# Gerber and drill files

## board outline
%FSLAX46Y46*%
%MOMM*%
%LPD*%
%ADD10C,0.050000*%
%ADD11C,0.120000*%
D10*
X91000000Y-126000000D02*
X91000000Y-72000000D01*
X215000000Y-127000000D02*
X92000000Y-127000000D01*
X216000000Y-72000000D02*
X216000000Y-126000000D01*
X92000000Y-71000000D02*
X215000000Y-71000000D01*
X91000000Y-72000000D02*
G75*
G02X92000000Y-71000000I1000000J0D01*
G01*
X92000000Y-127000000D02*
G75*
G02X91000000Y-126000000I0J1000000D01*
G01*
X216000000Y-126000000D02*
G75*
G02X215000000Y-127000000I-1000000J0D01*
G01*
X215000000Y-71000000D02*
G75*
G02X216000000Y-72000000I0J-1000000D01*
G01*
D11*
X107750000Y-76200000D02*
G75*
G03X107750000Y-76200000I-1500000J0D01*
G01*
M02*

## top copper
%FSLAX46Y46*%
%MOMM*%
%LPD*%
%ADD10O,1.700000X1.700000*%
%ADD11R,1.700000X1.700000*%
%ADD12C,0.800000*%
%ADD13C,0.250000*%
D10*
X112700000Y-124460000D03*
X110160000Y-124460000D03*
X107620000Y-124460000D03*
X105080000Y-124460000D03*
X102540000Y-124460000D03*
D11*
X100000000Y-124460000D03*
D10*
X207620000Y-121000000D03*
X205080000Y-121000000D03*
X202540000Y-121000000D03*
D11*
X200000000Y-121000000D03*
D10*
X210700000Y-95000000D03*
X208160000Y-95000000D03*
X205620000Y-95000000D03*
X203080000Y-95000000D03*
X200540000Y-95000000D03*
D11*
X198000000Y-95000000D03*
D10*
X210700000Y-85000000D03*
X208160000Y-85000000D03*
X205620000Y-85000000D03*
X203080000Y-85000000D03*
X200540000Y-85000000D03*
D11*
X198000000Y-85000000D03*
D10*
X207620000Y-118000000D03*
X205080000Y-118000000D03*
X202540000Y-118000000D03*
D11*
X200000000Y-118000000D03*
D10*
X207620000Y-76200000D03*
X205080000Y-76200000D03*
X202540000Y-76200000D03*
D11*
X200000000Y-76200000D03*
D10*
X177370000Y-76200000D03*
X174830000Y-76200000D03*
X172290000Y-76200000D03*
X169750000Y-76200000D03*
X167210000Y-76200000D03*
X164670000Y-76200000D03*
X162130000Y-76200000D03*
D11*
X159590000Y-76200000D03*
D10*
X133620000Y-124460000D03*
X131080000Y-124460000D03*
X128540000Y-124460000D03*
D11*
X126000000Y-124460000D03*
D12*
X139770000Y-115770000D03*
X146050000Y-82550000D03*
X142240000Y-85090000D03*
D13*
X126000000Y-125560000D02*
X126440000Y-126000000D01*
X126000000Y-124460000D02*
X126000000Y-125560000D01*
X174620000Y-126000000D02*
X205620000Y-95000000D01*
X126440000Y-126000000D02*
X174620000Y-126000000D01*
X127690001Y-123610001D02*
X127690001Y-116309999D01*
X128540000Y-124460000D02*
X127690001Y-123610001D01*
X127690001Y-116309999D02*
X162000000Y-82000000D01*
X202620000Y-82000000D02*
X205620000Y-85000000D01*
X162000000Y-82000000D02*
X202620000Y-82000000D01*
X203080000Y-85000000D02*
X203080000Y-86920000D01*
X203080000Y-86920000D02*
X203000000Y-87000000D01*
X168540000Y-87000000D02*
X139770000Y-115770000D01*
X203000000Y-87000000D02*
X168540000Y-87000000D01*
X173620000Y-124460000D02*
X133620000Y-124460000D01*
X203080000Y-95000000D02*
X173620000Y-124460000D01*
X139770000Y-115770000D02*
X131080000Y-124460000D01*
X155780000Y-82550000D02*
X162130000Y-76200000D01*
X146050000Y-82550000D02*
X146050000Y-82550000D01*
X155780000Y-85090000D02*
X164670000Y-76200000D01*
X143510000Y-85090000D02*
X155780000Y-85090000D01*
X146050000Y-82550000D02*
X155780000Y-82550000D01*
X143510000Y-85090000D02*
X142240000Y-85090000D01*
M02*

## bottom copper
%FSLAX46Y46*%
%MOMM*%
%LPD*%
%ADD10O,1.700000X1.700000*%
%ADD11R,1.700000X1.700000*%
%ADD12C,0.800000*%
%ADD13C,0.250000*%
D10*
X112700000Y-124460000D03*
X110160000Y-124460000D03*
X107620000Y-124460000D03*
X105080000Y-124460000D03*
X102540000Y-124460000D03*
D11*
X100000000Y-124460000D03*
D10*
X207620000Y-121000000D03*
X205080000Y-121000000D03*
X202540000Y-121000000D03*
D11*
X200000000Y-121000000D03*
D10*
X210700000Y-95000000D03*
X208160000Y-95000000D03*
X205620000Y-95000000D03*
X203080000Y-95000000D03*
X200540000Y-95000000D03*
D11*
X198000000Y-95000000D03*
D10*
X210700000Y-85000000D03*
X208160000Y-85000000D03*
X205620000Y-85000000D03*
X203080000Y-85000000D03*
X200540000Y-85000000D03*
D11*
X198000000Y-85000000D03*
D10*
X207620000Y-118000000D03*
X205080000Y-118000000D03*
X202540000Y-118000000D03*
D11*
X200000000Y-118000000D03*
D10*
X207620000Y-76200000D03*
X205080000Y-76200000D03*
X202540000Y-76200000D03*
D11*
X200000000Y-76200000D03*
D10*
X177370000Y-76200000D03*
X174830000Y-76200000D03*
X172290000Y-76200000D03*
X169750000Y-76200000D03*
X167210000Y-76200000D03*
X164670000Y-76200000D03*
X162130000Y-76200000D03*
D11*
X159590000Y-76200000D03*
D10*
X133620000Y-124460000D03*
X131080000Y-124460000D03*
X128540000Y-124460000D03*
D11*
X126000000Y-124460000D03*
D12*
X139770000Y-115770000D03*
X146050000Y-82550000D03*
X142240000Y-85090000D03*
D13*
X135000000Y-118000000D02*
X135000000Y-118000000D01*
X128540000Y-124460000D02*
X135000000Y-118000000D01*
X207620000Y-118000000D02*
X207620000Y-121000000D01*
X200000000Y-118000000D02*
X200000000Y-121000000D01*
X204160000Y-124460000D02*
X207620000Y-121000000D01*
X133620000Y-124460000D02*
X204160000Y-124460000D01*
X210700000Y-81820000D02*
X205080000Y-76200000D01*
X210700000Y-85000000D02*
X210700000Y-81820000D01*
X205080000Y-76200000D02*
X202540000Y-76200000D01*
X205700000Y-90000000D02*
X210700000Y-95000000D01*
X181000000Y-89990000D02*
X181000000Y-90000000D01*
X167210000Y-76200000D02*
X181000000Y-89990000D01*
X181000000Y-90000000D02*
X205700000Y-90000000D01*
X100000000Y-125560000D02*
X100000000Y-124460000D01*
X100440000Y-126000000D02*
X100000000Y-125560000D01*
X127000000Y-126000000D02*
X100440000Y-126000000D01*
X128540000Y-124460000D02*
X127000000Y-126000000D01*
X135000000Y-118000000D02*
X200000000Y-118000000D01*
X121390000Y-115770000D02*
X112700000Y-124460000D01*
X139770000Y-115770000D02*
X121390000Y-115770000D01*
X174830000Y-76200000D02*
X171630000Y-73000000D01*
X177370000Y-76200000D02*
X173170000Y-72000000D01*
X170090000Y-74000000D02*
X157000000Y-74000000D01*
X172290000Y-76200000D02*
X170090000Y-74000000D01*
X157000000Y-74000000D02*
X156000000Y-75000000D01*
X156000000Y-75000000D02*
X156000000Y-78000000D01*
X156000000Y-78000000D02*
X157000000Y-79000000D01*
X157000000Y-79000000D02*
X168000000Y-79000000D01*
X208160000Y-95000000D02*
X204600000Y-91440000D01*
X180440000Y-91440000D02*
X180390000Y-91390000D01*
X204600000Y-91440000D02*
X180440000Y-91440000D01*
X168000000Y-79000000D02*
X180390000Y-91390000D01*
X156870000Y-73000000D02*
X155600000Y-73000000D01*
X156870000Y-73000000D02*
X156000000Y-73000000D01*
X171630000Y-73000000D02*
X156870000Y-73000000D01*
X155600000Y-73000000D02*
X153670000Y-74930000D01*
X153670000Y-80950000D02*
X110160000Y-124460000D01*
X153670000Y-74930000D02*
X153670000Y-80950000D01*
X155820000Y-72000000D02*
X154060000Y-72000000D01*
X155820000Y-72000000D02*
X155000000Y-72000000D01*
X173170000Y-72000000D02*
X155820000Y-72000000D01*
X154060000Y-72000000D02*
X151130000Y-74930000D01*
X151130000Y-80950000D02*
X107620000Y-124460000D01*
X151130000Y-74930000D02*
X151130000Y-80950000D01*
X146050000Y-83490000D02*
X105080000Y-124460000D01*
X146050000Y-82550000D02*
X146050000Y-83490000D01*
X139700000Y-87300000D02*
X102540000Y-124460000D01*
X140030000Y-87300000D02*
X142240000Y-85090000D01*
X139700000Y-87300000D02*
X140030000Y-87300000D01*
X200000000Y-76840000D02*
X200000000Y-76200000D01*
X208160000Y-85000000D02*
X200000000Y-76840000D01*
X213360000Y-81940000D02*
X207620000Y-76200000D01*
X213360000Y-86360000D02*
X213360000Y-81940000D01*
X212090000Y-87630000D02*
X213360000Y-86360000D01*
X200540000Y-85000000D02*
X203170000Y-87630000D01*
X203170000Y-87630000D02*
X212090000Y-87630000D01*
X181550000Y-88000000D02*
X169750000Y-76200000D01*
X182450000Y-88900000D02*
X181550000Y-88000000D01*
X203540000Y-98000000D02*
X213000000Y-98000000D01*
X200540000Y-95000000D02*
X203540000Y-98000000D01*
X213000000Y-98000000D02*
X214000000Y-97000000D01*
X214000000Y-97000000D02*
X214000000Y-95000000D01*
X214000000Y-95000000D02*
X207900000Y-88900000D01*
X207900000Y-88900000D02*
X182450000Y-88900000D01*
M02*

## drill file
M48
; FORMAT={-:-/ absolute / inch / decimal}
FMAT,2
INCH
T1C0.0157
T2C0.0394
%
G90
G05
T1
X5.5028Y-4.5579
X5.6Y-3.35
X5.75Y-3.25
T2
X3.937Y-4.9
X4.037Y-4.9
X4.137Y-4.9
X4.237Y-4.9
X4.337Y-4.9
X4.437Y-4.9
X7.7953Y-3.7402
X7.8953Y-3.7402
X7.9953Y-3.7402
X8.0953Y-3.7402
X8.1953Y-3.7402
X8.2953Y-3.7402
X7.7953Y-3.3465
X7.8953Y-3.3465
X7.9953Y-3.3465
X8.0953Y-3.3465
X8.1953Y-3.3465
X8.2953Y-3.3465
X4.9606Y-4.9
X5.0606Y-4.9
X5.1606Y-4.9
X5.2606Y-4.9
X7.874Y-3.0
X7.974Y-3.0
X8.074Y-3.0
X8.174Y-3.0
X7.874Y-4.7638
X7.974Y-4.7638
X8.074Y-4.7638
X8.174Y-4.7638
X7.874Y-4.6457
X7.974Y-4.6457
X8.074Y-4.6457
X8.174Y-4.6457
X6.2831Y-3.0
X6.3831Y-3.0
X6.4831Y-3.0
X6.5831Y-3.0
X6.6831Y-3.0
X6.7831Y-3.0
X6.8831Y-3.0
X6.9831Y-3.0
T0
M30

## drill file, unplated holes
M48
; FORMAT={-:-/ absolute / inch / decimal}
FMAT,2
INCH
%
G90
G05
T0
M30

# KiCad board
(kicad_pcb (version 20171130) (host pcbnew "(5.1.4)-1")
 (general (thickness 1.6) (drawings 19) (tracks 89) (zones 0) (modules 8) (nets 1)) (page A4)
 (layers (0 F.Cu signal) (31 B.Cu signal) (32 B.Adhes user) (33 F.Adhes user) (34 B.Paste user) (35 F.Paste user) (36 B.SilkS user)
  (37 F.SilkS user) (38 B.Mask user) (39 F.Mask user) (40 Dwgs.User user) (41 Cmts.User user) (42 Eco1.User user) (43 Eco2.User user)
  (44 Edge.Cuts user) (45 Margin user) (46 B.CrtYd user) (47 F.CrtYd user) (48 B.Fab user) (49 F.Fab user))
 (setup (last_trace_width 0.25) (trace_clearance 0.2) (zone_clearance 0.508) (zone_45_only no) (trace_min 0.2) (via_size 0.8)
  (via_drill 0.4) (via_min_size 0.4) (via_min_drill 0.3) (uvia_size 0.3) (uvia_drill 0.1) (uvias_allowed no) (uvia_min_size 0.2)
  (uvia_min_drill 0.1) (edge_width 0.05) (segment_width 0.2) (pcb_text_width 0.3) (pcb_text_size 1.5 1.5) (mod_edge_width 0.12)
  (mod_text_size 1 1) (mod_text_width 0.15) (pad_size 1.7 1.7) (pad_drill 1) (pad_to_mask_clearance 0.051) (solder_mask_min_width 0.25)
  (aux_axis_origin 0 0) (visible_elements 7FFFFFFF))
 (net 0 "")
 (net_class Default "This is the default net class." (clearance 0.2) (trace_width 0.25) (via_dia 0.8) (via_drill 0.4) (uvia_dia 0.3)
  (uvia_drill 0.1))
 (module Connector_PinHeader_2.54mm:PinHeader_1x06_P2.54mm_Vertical (layer B.Cu) (at 100 124.46 270)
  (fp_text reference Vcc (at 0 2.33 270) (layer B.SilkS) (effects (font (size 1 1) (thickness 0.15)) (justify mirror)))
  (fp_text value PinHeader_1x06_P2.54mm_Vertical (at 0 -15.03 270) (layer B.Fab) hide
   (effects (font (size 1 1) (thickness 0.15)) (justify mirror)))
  (pad 6 thru_hole oval (at 0 -12.7 270) (size 1.7 1.7) (drill 1) (layers *.Cu *.Mask))
  (pad 5 thru_hole oval (at 0 -10.16 270) (size 1.7 1.7) (drill 1) (layers *.Cu *.Mask))
  (pad 4 thru_hole oval (at 0 -7.62 270) (size 1.7 1.7) (drill 1) (layers *.Cu *.Mask))
  (pad 3 thru_hole oval (at 0 -5.08 270) (size 1.7 1.7) (drill 1) (layers *.Cu *.Mask))
  (pad 2 thru_hole oval (at 0 -2.54 270) (size 1.7 1.7) (drill 1) (layers *.Cu *.Mask))
  (pad 1 thru_hole rect (at 0 0 270) (size 1.7 1.7) (drill 1) (layers *.Cu *.Mask)))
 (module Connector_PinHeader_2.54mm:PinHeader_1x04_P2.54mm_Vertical (layer F.Cu) (at 200 121 90)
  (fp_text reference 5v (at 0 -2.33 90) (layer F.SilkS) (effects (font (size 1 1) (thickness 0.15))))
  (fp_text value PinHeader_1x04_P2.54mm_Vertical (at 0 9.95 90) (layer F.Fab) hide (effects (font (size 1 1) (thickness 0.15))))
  (pad 4 thru_hole oval (at 0 7.62 90) (size 1.7 1.7) (drill 1) (layers *.Cu *.Mask))
  (pad 3 thru_hole oval (at 0 5.08 90) (size 1.7 1.7) (drill 1) (layers *.Cu *.Mask))
  (pad 2 thru_hole oval (at 0 2.54 90) (size 1.7 1.7) (drill 1) (layers *.Cu *.Mask))
  (pad 1 thru_hole rect (at 0 0 90) (size 1.7 1.7) (drill 1) (layers *.Cu *.Mask)))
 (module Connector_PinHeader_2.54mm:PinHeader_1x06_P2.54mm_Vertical (layer B.Cu) (at 198 95 270)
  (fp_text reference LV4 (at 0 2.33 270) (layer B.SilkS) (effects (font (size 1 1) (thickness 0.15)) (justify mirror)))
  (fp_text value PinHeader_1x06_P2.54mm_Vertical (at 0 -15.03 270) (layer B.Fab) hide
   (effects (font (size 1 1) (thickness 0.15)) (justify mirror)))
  (pad 6 thru_hole oval (at 0 -12.7 270) (size 1.7 1.7) (drill 1) (layers *.Cu *.Mask))
  (pad 5 thru_hole oval (at 0 -10.16 270) (size 1.7 1.7) (drill 1) (layers *.Cu *.Mask))
  (pad 4 thru_hole oval (at 0 -7.62 270) (size 1.7 1.7) (drill 1) (layers *.Cu *.Mask))
  (pad 3 thru_hole oval (at 0 -5.08 270) (size 1.7 1.7) (drill 1) (layers *.Cu *.Mask))
  (pad 2 thru_hole oval (at 0 -2.54 270) (size 1.7 1.7) (drill 1) (layers *.Cu *.Mask))
  (pad 1 thru_hole rect (at 0 0 270) (size 1.7 1.7) (drill 1) (layers *.Cu *.Mask)))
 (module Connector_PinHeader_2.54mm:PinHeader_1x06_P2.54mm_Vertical (layer B.Cu) (at 198 85 270)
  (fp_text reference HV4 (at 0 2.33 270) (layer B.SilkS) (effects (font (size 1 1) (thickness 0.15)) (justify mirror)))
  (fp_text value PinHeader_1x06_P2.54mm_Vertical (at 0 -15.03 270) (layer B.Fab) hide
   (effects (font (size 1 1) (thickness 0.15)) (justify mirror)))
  (pad 6 thru_hole oval (at 0 -12.7 270) (size 1.7 1.7) (drill 1) (layers *.Cu *.Mask))
  (pad 5 thru_hole oval (at 0 -10.16 270) (size 1.7 1.7) (drill 1) (layers *.Cu *.Mask))
  (pad 4 thru_hole oval (at 0 -7.62 270) (size 1.7 1.7) (drill 1) (layers *.Cu *.Mask))
  (pad 3 thru_hole oval (at 0 -5.08 270) (size 1.7 1.7) (drill 1) (layers *.Cu *.Mask))
  (pad 2 thru_hole oval (at 0 -2.54 270) (size 1.7 1.7) (drill 1) (layers *.Cu *.Mask))
  (pad 1 thru_hole rect (at 0 0 270) (size 1.7 1.7) (drill 1) (layers *.Cu *.Mask)))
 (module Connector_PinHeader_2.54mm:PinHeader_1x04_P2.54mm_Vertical (layer F.Cu) (at 200 118 90)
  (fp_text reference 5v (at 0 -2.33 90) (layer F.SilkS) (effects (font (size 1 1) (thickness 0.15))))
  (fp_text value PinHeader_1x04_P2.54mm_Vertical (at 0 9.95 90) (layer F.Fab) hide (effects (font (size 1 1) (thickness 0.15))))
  (pad 4 thru_hole oval (at 0 7.62 90) (size 1.7 1.7) (drill 1) (layers *.Cu *.Mask))
  (pad 3 thru_hole oval (at 0 5.08 90) (size 1.7 1.7) (drill 1) (layers *.Cu *.Mask))
  (pad 2 thru_hole oval (at 0 2.54 90) (size 1.7 1.7) (drill 1) (layers *.Cu *.Mask))
  (pad 1 thru_hole rect (at 0 0 90) (size 1.7 1.7) (drill 1) (layers *.Cu *.Mask)))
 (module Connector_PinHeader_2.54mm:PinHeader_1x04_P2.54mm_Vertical (layer F.Cu) (at 200 76.2 90)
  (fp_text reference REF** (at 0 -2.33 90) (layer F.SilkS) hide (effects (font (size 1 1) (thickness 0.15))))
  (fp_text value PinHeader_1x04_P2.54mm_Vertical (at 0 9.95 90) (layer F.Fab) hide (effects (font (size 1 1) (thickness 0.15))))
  (pad 4 thru_hole oval (at 0 7.62 90) (size 1.7 1.7) (drill 1) (layers *.Cu *.Mask))
  (pad 3 thru_hole oval (at 0 5.08 90) (size 1.7 1.7) (drill 1) (layers *.Cu *.Mask))
  (pad 2 thru_hole oval (at 0 2.54 90) (size 1.7 1.7) (drill 1) (layers *.Cu *.Mask))
  (pad 1 thru_hole rect (at 0 0 90) (size 1.7 1.7) (drill 1) (layers *.Cu *.Mask)))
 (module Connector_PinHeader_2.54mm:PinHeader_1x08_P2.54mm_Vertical (layer F.Cu) (at 159.59 76.2 90)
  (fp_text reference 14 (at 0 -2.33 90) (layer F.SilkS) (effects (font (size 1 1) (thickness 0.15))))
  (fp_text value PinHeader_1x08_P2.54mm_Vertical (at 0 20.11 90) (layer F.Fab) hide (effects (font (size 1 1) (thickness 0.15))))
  (pad 8 thru_hole oval (at 0 17.78 90) (size 1.7 1.7) (drill 1) (layers *.Cu *.Mask))
  (pad 7 thru_hole oval (at 0 15.24 90) (size 1.7 1.7) (drill 1) (layers *.Cu *.Mask))
  (pad 6 thru_hole oval (at 0 12.7 90) (size 1.7 1.7) (drill 1) (layers *.Cu *.Mask))
  (pad 5 thru_hole oval (at 0 10.16 90) (size 1.7 1.7) (drill 1) (layers *.Cu *.Mask))
  (pad 4 thru_hole oval (at 0 7.62 90) (size 1.7 1.7) (drill 1) (layers *.Cu *.Mask))
  (pad 3 thru_hole oval (at 0 5.08 90) (size 1.7 1.7) (drill 1) (layers *.Cu *.Mask))
  (pad 2 thru_hole oval (at 0 2.54 90) (size 1.7 1.7) (drill 1) (layers *.Cu *.Mask))
  (pad 1 thru_hole rect (at 0 0 90) (size 1.7 1.7) (drill 1) (layers *.Cu *.Mask)))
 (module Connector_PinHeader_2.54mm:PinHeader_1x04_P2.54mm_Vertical (layer F.Cu) (at 126 124.46 90)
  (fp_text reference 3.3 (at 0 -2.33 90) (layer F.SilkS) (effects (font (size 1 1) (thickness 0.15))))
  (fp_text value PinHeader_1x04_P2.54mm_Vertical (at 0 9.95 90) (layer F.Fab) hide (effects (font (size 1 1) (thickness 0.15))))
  (pad 4 thru_hole oval (at 0 7.62 90) (size 1.7 1.7) (drill 1) (layers *.Cu *.Mask))
  (pad 3 thru_hole oval (at 0 5.08 90) (size 1.7 1.7) (drill 1) (layers *.Cu *.Mask))
  (pad 2 thru_hole oval (at 0 2.54 90) (size 1.7 1.7) (drill 1) (layers *.Cu *.Mask))
  (pad 1 thru_hole rect (at 0 0 90) (size 1.7 1.7) (drill 1) (layers *.Cu *.Mask)))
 (gr_line (start 91 126) (end 91 72) (layer Edge.Cuts) (width 0.05))
 (gr_line (start 215 127) (end 92 127) (layer Edge.Cuts) (width 0.05))
 (gr_line (start 216 72) (end 216 126) (layer Edge.Cuts) (width 0.05))
 (gr_line (start 92 71) (end 215 71) (layer Edge.Cuts) (width 0.05))
 (gr_arc (start 92 72) (end 92 71) (angle -90) (layer Edge.Cuts) (width 0.05))
 (gr_arc (start 92 126) (end 91 126) (angle -90) (layer Edge.Cuts) (width 0.05))
 (gr_arc (start 215 126) (end 215 127) (angle -90) (layer Edge.Cuts) (width 0.05))
 (gr_arc (start 215 72) (end 216 72) (angle -90) (layer Edge.Cuts) (width 0.05))
 (gr_circle (center 106.25 76.2) (end 107.75 76.2) (layer Edge.Cuts) (width 0.12))
 (segment (start 126 125.56) (end 126.44 126) (width 0.25) (layer F.Cu) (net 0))
 (segment (start 126 124.46) (end 126 125.56) (width 0.25) (layer F.Cu) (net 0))
 (segment (start 174.62 126) (end 205.62 95) (width 0.25) (layer F.Cu) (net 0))
 (segment (start 126.44 126) (end 174.62 126) (width 0.25) (layer F.Cu) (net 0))
 (segment (start 127.690001 123.610001) (end 127.690001 116.309999) (width 0.25) (layer F.Cu) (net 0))
 (segment (start 128.54 124.46) (end 127.690001 123.610001) (width 0.25) (layer F.Cu) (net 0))
 (segment (start 127.690001 116.309999) (end 162 82) (width 0.25) (layer F.Cu) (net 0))
 (segment (start 202.62 82) (end 205.62 85) (width 0.25) (layer F.Cu) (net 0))
 (segment (start 162 82) (end 202.62 82) (width 0.25) (layer F.Cu) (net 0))
 (segment (start 203.08 85) (end 203.08 86.92) (width 0.25) (layer F.Cu) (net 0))
 (segment (start 203.08 86.92) (end 203 87) (width 0.25) (layer F.Cu) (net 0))
 (segment (start 168.54 87) (end 139.77 115.77) (width 0.25) (layer F.Cu) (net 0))
 (segment (start 203 87) (end 168.54 87) (width 0.25) (layer F.Cu) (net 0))
 (segment (start 173.62 124.46) (end 133.62 124.46) (width 0.25) (layer F.Cu) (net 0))
 (segment (start 203.08 95) (end 173.62 124.46) (width 0.25) (layer F.Cu) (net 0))
 (segment (start 135 118) (end 135 118) (width 0.25) (layer B.Cu) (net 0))
 (segment (start 128.54 124.46) (end 135 118) (width 0.25) (layer B.Cu) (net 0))
 (segment (start 207.62 118) (end 207.62 121) (width 0.25) (layer B.Cu) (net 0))
 (segment (start 200 118) (end 200 121) (width 0.25) (layer B.Cu) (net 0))
 (segment (start 204.16 124.46) (end 207.62 121) (width 0.25) (layer B.Cu) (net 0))
 (segment (start 133.62 124.46) (end 204.16 124.46) (width 0.25) (layer B.Cu) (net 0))
 (segment (start 210.7 81.82) (end 205.08 76.2) (width 0.25) (layer B.Cu) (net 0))
 (segment (start 210.7 85) (end 210.7 81.82) (width 0.25) (layer B.Cu) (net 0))
 (segment (start 205.08 76.2) (end 202.54 76.2) (width 0.25) (layer B.Cu) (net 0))
 (segment (start 205.7 90) (end 210.7 95) (width 0.25) (layer B.Cu) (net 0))
 (segment (start 181 89.99) (end 181 90) (width 0.25) (layer B.Cu) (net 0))
 (segment (start 167.21 76.2) (end 181 89.99) (width 0.25) (layer B.Cu) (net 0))
 (segment (start 181 90) (end 205.7 90) (width 0.25) (layer B.Cu) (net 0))
 (segment (start 100 125.56) (end 100 124.46) (width 0.25) (layer B.Cu) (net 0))
 (segment (start 100.44 126) (end 100 125.56) (width 0.25) (layer B.Cu) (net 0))
 (segment (start 127 126) (end 100.44 126) (width 0.25) (layer B.Cu) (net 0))
 (segment (start 128.54 124.46) (end 127 126) (width 0.25) (layer B.Cu) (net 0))
 (segment (start 135 118) (end 200 118) (width 0.25) (layer B.Cu) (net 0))
 (segment (start 139.77 115.77) (end 131.08 124.46) (width 0.25) (layer F.Cu) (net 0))
 (via (at 139.77 115.77) (size 0.8) (drill 0.4) (layers F.Cu B.Cu) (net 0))
 (segment (start 121.39 115.77) (end 112.7 124.46) (width 0.25) (layer B.Cu) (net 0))
 (segment (start 139.77 115.77) (end 121.39 115.77) (width 0.25) (layer B.Cu) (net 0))
 (segment (start 174.83 76.2) (end 171.63 73) (width 0.25) (layer B.Cu) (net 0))
 (segment (start 177.37 76.2) (end 173.17 72) (width 0.25) (layer B.Cu) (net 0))
 (segment (start 170.09 74) (end 157 74) (width 0.25) (layer B.Cu) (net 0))
 (segment (start 172.29 76.2) (end 170.09 74) (width 0.25) (layer B.Cu) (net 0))
 (segment (start 157 74) (end 156 75) (width 0.25) (layer B.Cu) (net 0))
 (segment (start 156 75) (end 156 78) (width 0.25) (layer B.Cu) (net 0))
 (segment (start 156 78) (end 157 79) (width 0.25) (layer B.Cu) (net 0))
 (segment (start 157 79) (end 168 79) (width 0.25) (layer B.Cu) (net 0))
 (segment (start 208.16 95) (end 204.6 91.44) (width 0.25) (layer B.Cu) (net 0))
 (segment (start 180.44 91.44) (end 180.39 91.39) (width 0.25) (layer B.Cu) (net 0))
 (segment (start 204.6 91.44) (end 180.44 91.44) (width 0.25) (layer B.Cu) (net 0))
 (segment (start 168 79) (end 180.39 91.39) (width 0.25) (layer B.Cu) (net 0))
 (segment (start 156.87 73) (end 155.6 73) (width 0.25) (layer B.Cu) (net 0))
 (segment (start 156.87 73) (end 156 73) (width 0.25) (layer B.Cu) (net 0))
 (segment (start 171.63 73) (end 156.87 73) (width 0.25) (layer B.Cu) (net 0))
 (segment (start 155.6 73) (end 153.67 74.93) (width 0.25) (layer B.Cu) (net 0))
 (segment (start 153.67 80.95) (end 110.16 124.46) (width 0.25) (layer B.Cu) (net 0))
 (segment (start 153.67 74.93) (end 153.67 80.95) (width 0.25) (layer B.Cu) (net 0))
 (segment (start 155.82 72) (end 154.06 72) (width 0.25) (layer B.Cu) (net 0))
 (segment (start 155.82 72) (end 155 72) (width 0.25) (layer B.Cu) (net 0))
 (segment (start 173.17 72) (end 155.82 72) (width 0.25) (layer B.Cu) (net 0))
 (segment (start 154.06 72) (end 151.13 74.93) (width 0.25) (layer B.Cu) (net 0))
 (segment (start 151.13 80.95) (end 107.62 124.46) (width 0.25) (layer B.Cu) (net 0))
 (segment (start 151.13 74.93) (end 151.13 80.95) (width 0.25) (layer B.Cu) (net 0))
 (segment (start 155.78 82.55) (end 162.13 76.2) (width 0.25) (layer F.Cu) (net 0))
 (segment (start 146.05 82.55) (end 146.05 82.55) (width 0.25) (layer F.Cu) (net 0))
 (segment (start 155.78 85.09) (end 164.67 76.2) (width 0.25) (layer F.Cu) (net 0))
 (segment (start 143.51 85.09) (end 155.78 85.09) (width 0.25) (layer F.Cu) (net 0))
 (segment (start 146.05 82.55) (end 155.78 82.55) (width 0.25) (layer F.Cu) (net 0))
 (via (at 146.05 82.55) (size 0.8) (drill 0.4) (layers F.Cu B.Cu) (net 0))
 (segment (start 143.51 85.09) (end 142.24 85.09) (width 0.25) (layer F.Cu) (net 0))
 (segment (start 146.05 83.49) (end 105.08 124.46) (width 0.25) (layer B.Cu) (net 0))
 (segment (start 146.05 82.55) (end 146.05 83.49) (width 0.25) (layer B.Cu) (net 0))
 (segment (start 139.7 87.3) (end 102.54 124.46) (width 0.25) (layer B.Cu) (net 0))
 (via (at 142.24 85.09) (size 0.8) (drill 0.4) (layers F.Cu B.Cu) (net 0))
 (segment (start 140.03 87.3) (end 142.24 85.09) (width 0.25) (layer B.Cu) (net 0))
 (segment (start 139.7 87.3) (end 140.03 87.3) (width 0.25) (layer B.Cu) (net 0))
 (segment (start 200 76.84) (end 200 76.2) (width 0.25) (layer B.Cu) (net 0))
 (segment (start 208.16 85) (end 200 76.84) (width 0.25) (layer B.Cu) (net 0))
 (segment (start 213.36 81.94) (end 207.62 76.2) (width 0.25) (layer B.Cu) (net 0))
 (segment (start 213.36 86.36) (end 213.36 81.94) (width 0.25) (layer B.Cu) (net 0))
 (segment (start 212.09 87.63) (end 213.36 86.36) (width 0.25) (layer B.Cu) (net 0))
 (segment (start 200.54 85) (end 203.17 87.63) (width 0.25) (layer B.Cu) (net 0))
 (segment (start 203.17 87.63) (end 212.09 87.63) (width 0.25) (layer B.Cu) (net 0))
 (segment (start 181.55 88) (end 169.75 76.2) (width 0.25) (layer B.Cu) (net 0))
 (segment (start 182.45 88.9) (end 181.55 88) (width 0.25) (layer B.Cu) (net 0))
 (segment (start 203.54 98) (end 213 98) (width 0.25) (layer B.Cu) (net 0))
 (segment (start 200.54 95) (end 203.54 98) (width 0.25) (layer B.Cu) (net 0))
 (segment (start 213 98) (end 214 97) (width 0.25) (layer B.Cu) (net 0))
 (segment (start 214 97) (end 214 95) (width 0.25) (layer B.Cu) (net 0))
 (segment (start 214 95) (end 207.9 88.9) (width 0.25) (layer B.Cu) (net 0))
 (segment (start 207.9 88.9) (end 182.45 88.9) (width 0.25) (layer B.Cu) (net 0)))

